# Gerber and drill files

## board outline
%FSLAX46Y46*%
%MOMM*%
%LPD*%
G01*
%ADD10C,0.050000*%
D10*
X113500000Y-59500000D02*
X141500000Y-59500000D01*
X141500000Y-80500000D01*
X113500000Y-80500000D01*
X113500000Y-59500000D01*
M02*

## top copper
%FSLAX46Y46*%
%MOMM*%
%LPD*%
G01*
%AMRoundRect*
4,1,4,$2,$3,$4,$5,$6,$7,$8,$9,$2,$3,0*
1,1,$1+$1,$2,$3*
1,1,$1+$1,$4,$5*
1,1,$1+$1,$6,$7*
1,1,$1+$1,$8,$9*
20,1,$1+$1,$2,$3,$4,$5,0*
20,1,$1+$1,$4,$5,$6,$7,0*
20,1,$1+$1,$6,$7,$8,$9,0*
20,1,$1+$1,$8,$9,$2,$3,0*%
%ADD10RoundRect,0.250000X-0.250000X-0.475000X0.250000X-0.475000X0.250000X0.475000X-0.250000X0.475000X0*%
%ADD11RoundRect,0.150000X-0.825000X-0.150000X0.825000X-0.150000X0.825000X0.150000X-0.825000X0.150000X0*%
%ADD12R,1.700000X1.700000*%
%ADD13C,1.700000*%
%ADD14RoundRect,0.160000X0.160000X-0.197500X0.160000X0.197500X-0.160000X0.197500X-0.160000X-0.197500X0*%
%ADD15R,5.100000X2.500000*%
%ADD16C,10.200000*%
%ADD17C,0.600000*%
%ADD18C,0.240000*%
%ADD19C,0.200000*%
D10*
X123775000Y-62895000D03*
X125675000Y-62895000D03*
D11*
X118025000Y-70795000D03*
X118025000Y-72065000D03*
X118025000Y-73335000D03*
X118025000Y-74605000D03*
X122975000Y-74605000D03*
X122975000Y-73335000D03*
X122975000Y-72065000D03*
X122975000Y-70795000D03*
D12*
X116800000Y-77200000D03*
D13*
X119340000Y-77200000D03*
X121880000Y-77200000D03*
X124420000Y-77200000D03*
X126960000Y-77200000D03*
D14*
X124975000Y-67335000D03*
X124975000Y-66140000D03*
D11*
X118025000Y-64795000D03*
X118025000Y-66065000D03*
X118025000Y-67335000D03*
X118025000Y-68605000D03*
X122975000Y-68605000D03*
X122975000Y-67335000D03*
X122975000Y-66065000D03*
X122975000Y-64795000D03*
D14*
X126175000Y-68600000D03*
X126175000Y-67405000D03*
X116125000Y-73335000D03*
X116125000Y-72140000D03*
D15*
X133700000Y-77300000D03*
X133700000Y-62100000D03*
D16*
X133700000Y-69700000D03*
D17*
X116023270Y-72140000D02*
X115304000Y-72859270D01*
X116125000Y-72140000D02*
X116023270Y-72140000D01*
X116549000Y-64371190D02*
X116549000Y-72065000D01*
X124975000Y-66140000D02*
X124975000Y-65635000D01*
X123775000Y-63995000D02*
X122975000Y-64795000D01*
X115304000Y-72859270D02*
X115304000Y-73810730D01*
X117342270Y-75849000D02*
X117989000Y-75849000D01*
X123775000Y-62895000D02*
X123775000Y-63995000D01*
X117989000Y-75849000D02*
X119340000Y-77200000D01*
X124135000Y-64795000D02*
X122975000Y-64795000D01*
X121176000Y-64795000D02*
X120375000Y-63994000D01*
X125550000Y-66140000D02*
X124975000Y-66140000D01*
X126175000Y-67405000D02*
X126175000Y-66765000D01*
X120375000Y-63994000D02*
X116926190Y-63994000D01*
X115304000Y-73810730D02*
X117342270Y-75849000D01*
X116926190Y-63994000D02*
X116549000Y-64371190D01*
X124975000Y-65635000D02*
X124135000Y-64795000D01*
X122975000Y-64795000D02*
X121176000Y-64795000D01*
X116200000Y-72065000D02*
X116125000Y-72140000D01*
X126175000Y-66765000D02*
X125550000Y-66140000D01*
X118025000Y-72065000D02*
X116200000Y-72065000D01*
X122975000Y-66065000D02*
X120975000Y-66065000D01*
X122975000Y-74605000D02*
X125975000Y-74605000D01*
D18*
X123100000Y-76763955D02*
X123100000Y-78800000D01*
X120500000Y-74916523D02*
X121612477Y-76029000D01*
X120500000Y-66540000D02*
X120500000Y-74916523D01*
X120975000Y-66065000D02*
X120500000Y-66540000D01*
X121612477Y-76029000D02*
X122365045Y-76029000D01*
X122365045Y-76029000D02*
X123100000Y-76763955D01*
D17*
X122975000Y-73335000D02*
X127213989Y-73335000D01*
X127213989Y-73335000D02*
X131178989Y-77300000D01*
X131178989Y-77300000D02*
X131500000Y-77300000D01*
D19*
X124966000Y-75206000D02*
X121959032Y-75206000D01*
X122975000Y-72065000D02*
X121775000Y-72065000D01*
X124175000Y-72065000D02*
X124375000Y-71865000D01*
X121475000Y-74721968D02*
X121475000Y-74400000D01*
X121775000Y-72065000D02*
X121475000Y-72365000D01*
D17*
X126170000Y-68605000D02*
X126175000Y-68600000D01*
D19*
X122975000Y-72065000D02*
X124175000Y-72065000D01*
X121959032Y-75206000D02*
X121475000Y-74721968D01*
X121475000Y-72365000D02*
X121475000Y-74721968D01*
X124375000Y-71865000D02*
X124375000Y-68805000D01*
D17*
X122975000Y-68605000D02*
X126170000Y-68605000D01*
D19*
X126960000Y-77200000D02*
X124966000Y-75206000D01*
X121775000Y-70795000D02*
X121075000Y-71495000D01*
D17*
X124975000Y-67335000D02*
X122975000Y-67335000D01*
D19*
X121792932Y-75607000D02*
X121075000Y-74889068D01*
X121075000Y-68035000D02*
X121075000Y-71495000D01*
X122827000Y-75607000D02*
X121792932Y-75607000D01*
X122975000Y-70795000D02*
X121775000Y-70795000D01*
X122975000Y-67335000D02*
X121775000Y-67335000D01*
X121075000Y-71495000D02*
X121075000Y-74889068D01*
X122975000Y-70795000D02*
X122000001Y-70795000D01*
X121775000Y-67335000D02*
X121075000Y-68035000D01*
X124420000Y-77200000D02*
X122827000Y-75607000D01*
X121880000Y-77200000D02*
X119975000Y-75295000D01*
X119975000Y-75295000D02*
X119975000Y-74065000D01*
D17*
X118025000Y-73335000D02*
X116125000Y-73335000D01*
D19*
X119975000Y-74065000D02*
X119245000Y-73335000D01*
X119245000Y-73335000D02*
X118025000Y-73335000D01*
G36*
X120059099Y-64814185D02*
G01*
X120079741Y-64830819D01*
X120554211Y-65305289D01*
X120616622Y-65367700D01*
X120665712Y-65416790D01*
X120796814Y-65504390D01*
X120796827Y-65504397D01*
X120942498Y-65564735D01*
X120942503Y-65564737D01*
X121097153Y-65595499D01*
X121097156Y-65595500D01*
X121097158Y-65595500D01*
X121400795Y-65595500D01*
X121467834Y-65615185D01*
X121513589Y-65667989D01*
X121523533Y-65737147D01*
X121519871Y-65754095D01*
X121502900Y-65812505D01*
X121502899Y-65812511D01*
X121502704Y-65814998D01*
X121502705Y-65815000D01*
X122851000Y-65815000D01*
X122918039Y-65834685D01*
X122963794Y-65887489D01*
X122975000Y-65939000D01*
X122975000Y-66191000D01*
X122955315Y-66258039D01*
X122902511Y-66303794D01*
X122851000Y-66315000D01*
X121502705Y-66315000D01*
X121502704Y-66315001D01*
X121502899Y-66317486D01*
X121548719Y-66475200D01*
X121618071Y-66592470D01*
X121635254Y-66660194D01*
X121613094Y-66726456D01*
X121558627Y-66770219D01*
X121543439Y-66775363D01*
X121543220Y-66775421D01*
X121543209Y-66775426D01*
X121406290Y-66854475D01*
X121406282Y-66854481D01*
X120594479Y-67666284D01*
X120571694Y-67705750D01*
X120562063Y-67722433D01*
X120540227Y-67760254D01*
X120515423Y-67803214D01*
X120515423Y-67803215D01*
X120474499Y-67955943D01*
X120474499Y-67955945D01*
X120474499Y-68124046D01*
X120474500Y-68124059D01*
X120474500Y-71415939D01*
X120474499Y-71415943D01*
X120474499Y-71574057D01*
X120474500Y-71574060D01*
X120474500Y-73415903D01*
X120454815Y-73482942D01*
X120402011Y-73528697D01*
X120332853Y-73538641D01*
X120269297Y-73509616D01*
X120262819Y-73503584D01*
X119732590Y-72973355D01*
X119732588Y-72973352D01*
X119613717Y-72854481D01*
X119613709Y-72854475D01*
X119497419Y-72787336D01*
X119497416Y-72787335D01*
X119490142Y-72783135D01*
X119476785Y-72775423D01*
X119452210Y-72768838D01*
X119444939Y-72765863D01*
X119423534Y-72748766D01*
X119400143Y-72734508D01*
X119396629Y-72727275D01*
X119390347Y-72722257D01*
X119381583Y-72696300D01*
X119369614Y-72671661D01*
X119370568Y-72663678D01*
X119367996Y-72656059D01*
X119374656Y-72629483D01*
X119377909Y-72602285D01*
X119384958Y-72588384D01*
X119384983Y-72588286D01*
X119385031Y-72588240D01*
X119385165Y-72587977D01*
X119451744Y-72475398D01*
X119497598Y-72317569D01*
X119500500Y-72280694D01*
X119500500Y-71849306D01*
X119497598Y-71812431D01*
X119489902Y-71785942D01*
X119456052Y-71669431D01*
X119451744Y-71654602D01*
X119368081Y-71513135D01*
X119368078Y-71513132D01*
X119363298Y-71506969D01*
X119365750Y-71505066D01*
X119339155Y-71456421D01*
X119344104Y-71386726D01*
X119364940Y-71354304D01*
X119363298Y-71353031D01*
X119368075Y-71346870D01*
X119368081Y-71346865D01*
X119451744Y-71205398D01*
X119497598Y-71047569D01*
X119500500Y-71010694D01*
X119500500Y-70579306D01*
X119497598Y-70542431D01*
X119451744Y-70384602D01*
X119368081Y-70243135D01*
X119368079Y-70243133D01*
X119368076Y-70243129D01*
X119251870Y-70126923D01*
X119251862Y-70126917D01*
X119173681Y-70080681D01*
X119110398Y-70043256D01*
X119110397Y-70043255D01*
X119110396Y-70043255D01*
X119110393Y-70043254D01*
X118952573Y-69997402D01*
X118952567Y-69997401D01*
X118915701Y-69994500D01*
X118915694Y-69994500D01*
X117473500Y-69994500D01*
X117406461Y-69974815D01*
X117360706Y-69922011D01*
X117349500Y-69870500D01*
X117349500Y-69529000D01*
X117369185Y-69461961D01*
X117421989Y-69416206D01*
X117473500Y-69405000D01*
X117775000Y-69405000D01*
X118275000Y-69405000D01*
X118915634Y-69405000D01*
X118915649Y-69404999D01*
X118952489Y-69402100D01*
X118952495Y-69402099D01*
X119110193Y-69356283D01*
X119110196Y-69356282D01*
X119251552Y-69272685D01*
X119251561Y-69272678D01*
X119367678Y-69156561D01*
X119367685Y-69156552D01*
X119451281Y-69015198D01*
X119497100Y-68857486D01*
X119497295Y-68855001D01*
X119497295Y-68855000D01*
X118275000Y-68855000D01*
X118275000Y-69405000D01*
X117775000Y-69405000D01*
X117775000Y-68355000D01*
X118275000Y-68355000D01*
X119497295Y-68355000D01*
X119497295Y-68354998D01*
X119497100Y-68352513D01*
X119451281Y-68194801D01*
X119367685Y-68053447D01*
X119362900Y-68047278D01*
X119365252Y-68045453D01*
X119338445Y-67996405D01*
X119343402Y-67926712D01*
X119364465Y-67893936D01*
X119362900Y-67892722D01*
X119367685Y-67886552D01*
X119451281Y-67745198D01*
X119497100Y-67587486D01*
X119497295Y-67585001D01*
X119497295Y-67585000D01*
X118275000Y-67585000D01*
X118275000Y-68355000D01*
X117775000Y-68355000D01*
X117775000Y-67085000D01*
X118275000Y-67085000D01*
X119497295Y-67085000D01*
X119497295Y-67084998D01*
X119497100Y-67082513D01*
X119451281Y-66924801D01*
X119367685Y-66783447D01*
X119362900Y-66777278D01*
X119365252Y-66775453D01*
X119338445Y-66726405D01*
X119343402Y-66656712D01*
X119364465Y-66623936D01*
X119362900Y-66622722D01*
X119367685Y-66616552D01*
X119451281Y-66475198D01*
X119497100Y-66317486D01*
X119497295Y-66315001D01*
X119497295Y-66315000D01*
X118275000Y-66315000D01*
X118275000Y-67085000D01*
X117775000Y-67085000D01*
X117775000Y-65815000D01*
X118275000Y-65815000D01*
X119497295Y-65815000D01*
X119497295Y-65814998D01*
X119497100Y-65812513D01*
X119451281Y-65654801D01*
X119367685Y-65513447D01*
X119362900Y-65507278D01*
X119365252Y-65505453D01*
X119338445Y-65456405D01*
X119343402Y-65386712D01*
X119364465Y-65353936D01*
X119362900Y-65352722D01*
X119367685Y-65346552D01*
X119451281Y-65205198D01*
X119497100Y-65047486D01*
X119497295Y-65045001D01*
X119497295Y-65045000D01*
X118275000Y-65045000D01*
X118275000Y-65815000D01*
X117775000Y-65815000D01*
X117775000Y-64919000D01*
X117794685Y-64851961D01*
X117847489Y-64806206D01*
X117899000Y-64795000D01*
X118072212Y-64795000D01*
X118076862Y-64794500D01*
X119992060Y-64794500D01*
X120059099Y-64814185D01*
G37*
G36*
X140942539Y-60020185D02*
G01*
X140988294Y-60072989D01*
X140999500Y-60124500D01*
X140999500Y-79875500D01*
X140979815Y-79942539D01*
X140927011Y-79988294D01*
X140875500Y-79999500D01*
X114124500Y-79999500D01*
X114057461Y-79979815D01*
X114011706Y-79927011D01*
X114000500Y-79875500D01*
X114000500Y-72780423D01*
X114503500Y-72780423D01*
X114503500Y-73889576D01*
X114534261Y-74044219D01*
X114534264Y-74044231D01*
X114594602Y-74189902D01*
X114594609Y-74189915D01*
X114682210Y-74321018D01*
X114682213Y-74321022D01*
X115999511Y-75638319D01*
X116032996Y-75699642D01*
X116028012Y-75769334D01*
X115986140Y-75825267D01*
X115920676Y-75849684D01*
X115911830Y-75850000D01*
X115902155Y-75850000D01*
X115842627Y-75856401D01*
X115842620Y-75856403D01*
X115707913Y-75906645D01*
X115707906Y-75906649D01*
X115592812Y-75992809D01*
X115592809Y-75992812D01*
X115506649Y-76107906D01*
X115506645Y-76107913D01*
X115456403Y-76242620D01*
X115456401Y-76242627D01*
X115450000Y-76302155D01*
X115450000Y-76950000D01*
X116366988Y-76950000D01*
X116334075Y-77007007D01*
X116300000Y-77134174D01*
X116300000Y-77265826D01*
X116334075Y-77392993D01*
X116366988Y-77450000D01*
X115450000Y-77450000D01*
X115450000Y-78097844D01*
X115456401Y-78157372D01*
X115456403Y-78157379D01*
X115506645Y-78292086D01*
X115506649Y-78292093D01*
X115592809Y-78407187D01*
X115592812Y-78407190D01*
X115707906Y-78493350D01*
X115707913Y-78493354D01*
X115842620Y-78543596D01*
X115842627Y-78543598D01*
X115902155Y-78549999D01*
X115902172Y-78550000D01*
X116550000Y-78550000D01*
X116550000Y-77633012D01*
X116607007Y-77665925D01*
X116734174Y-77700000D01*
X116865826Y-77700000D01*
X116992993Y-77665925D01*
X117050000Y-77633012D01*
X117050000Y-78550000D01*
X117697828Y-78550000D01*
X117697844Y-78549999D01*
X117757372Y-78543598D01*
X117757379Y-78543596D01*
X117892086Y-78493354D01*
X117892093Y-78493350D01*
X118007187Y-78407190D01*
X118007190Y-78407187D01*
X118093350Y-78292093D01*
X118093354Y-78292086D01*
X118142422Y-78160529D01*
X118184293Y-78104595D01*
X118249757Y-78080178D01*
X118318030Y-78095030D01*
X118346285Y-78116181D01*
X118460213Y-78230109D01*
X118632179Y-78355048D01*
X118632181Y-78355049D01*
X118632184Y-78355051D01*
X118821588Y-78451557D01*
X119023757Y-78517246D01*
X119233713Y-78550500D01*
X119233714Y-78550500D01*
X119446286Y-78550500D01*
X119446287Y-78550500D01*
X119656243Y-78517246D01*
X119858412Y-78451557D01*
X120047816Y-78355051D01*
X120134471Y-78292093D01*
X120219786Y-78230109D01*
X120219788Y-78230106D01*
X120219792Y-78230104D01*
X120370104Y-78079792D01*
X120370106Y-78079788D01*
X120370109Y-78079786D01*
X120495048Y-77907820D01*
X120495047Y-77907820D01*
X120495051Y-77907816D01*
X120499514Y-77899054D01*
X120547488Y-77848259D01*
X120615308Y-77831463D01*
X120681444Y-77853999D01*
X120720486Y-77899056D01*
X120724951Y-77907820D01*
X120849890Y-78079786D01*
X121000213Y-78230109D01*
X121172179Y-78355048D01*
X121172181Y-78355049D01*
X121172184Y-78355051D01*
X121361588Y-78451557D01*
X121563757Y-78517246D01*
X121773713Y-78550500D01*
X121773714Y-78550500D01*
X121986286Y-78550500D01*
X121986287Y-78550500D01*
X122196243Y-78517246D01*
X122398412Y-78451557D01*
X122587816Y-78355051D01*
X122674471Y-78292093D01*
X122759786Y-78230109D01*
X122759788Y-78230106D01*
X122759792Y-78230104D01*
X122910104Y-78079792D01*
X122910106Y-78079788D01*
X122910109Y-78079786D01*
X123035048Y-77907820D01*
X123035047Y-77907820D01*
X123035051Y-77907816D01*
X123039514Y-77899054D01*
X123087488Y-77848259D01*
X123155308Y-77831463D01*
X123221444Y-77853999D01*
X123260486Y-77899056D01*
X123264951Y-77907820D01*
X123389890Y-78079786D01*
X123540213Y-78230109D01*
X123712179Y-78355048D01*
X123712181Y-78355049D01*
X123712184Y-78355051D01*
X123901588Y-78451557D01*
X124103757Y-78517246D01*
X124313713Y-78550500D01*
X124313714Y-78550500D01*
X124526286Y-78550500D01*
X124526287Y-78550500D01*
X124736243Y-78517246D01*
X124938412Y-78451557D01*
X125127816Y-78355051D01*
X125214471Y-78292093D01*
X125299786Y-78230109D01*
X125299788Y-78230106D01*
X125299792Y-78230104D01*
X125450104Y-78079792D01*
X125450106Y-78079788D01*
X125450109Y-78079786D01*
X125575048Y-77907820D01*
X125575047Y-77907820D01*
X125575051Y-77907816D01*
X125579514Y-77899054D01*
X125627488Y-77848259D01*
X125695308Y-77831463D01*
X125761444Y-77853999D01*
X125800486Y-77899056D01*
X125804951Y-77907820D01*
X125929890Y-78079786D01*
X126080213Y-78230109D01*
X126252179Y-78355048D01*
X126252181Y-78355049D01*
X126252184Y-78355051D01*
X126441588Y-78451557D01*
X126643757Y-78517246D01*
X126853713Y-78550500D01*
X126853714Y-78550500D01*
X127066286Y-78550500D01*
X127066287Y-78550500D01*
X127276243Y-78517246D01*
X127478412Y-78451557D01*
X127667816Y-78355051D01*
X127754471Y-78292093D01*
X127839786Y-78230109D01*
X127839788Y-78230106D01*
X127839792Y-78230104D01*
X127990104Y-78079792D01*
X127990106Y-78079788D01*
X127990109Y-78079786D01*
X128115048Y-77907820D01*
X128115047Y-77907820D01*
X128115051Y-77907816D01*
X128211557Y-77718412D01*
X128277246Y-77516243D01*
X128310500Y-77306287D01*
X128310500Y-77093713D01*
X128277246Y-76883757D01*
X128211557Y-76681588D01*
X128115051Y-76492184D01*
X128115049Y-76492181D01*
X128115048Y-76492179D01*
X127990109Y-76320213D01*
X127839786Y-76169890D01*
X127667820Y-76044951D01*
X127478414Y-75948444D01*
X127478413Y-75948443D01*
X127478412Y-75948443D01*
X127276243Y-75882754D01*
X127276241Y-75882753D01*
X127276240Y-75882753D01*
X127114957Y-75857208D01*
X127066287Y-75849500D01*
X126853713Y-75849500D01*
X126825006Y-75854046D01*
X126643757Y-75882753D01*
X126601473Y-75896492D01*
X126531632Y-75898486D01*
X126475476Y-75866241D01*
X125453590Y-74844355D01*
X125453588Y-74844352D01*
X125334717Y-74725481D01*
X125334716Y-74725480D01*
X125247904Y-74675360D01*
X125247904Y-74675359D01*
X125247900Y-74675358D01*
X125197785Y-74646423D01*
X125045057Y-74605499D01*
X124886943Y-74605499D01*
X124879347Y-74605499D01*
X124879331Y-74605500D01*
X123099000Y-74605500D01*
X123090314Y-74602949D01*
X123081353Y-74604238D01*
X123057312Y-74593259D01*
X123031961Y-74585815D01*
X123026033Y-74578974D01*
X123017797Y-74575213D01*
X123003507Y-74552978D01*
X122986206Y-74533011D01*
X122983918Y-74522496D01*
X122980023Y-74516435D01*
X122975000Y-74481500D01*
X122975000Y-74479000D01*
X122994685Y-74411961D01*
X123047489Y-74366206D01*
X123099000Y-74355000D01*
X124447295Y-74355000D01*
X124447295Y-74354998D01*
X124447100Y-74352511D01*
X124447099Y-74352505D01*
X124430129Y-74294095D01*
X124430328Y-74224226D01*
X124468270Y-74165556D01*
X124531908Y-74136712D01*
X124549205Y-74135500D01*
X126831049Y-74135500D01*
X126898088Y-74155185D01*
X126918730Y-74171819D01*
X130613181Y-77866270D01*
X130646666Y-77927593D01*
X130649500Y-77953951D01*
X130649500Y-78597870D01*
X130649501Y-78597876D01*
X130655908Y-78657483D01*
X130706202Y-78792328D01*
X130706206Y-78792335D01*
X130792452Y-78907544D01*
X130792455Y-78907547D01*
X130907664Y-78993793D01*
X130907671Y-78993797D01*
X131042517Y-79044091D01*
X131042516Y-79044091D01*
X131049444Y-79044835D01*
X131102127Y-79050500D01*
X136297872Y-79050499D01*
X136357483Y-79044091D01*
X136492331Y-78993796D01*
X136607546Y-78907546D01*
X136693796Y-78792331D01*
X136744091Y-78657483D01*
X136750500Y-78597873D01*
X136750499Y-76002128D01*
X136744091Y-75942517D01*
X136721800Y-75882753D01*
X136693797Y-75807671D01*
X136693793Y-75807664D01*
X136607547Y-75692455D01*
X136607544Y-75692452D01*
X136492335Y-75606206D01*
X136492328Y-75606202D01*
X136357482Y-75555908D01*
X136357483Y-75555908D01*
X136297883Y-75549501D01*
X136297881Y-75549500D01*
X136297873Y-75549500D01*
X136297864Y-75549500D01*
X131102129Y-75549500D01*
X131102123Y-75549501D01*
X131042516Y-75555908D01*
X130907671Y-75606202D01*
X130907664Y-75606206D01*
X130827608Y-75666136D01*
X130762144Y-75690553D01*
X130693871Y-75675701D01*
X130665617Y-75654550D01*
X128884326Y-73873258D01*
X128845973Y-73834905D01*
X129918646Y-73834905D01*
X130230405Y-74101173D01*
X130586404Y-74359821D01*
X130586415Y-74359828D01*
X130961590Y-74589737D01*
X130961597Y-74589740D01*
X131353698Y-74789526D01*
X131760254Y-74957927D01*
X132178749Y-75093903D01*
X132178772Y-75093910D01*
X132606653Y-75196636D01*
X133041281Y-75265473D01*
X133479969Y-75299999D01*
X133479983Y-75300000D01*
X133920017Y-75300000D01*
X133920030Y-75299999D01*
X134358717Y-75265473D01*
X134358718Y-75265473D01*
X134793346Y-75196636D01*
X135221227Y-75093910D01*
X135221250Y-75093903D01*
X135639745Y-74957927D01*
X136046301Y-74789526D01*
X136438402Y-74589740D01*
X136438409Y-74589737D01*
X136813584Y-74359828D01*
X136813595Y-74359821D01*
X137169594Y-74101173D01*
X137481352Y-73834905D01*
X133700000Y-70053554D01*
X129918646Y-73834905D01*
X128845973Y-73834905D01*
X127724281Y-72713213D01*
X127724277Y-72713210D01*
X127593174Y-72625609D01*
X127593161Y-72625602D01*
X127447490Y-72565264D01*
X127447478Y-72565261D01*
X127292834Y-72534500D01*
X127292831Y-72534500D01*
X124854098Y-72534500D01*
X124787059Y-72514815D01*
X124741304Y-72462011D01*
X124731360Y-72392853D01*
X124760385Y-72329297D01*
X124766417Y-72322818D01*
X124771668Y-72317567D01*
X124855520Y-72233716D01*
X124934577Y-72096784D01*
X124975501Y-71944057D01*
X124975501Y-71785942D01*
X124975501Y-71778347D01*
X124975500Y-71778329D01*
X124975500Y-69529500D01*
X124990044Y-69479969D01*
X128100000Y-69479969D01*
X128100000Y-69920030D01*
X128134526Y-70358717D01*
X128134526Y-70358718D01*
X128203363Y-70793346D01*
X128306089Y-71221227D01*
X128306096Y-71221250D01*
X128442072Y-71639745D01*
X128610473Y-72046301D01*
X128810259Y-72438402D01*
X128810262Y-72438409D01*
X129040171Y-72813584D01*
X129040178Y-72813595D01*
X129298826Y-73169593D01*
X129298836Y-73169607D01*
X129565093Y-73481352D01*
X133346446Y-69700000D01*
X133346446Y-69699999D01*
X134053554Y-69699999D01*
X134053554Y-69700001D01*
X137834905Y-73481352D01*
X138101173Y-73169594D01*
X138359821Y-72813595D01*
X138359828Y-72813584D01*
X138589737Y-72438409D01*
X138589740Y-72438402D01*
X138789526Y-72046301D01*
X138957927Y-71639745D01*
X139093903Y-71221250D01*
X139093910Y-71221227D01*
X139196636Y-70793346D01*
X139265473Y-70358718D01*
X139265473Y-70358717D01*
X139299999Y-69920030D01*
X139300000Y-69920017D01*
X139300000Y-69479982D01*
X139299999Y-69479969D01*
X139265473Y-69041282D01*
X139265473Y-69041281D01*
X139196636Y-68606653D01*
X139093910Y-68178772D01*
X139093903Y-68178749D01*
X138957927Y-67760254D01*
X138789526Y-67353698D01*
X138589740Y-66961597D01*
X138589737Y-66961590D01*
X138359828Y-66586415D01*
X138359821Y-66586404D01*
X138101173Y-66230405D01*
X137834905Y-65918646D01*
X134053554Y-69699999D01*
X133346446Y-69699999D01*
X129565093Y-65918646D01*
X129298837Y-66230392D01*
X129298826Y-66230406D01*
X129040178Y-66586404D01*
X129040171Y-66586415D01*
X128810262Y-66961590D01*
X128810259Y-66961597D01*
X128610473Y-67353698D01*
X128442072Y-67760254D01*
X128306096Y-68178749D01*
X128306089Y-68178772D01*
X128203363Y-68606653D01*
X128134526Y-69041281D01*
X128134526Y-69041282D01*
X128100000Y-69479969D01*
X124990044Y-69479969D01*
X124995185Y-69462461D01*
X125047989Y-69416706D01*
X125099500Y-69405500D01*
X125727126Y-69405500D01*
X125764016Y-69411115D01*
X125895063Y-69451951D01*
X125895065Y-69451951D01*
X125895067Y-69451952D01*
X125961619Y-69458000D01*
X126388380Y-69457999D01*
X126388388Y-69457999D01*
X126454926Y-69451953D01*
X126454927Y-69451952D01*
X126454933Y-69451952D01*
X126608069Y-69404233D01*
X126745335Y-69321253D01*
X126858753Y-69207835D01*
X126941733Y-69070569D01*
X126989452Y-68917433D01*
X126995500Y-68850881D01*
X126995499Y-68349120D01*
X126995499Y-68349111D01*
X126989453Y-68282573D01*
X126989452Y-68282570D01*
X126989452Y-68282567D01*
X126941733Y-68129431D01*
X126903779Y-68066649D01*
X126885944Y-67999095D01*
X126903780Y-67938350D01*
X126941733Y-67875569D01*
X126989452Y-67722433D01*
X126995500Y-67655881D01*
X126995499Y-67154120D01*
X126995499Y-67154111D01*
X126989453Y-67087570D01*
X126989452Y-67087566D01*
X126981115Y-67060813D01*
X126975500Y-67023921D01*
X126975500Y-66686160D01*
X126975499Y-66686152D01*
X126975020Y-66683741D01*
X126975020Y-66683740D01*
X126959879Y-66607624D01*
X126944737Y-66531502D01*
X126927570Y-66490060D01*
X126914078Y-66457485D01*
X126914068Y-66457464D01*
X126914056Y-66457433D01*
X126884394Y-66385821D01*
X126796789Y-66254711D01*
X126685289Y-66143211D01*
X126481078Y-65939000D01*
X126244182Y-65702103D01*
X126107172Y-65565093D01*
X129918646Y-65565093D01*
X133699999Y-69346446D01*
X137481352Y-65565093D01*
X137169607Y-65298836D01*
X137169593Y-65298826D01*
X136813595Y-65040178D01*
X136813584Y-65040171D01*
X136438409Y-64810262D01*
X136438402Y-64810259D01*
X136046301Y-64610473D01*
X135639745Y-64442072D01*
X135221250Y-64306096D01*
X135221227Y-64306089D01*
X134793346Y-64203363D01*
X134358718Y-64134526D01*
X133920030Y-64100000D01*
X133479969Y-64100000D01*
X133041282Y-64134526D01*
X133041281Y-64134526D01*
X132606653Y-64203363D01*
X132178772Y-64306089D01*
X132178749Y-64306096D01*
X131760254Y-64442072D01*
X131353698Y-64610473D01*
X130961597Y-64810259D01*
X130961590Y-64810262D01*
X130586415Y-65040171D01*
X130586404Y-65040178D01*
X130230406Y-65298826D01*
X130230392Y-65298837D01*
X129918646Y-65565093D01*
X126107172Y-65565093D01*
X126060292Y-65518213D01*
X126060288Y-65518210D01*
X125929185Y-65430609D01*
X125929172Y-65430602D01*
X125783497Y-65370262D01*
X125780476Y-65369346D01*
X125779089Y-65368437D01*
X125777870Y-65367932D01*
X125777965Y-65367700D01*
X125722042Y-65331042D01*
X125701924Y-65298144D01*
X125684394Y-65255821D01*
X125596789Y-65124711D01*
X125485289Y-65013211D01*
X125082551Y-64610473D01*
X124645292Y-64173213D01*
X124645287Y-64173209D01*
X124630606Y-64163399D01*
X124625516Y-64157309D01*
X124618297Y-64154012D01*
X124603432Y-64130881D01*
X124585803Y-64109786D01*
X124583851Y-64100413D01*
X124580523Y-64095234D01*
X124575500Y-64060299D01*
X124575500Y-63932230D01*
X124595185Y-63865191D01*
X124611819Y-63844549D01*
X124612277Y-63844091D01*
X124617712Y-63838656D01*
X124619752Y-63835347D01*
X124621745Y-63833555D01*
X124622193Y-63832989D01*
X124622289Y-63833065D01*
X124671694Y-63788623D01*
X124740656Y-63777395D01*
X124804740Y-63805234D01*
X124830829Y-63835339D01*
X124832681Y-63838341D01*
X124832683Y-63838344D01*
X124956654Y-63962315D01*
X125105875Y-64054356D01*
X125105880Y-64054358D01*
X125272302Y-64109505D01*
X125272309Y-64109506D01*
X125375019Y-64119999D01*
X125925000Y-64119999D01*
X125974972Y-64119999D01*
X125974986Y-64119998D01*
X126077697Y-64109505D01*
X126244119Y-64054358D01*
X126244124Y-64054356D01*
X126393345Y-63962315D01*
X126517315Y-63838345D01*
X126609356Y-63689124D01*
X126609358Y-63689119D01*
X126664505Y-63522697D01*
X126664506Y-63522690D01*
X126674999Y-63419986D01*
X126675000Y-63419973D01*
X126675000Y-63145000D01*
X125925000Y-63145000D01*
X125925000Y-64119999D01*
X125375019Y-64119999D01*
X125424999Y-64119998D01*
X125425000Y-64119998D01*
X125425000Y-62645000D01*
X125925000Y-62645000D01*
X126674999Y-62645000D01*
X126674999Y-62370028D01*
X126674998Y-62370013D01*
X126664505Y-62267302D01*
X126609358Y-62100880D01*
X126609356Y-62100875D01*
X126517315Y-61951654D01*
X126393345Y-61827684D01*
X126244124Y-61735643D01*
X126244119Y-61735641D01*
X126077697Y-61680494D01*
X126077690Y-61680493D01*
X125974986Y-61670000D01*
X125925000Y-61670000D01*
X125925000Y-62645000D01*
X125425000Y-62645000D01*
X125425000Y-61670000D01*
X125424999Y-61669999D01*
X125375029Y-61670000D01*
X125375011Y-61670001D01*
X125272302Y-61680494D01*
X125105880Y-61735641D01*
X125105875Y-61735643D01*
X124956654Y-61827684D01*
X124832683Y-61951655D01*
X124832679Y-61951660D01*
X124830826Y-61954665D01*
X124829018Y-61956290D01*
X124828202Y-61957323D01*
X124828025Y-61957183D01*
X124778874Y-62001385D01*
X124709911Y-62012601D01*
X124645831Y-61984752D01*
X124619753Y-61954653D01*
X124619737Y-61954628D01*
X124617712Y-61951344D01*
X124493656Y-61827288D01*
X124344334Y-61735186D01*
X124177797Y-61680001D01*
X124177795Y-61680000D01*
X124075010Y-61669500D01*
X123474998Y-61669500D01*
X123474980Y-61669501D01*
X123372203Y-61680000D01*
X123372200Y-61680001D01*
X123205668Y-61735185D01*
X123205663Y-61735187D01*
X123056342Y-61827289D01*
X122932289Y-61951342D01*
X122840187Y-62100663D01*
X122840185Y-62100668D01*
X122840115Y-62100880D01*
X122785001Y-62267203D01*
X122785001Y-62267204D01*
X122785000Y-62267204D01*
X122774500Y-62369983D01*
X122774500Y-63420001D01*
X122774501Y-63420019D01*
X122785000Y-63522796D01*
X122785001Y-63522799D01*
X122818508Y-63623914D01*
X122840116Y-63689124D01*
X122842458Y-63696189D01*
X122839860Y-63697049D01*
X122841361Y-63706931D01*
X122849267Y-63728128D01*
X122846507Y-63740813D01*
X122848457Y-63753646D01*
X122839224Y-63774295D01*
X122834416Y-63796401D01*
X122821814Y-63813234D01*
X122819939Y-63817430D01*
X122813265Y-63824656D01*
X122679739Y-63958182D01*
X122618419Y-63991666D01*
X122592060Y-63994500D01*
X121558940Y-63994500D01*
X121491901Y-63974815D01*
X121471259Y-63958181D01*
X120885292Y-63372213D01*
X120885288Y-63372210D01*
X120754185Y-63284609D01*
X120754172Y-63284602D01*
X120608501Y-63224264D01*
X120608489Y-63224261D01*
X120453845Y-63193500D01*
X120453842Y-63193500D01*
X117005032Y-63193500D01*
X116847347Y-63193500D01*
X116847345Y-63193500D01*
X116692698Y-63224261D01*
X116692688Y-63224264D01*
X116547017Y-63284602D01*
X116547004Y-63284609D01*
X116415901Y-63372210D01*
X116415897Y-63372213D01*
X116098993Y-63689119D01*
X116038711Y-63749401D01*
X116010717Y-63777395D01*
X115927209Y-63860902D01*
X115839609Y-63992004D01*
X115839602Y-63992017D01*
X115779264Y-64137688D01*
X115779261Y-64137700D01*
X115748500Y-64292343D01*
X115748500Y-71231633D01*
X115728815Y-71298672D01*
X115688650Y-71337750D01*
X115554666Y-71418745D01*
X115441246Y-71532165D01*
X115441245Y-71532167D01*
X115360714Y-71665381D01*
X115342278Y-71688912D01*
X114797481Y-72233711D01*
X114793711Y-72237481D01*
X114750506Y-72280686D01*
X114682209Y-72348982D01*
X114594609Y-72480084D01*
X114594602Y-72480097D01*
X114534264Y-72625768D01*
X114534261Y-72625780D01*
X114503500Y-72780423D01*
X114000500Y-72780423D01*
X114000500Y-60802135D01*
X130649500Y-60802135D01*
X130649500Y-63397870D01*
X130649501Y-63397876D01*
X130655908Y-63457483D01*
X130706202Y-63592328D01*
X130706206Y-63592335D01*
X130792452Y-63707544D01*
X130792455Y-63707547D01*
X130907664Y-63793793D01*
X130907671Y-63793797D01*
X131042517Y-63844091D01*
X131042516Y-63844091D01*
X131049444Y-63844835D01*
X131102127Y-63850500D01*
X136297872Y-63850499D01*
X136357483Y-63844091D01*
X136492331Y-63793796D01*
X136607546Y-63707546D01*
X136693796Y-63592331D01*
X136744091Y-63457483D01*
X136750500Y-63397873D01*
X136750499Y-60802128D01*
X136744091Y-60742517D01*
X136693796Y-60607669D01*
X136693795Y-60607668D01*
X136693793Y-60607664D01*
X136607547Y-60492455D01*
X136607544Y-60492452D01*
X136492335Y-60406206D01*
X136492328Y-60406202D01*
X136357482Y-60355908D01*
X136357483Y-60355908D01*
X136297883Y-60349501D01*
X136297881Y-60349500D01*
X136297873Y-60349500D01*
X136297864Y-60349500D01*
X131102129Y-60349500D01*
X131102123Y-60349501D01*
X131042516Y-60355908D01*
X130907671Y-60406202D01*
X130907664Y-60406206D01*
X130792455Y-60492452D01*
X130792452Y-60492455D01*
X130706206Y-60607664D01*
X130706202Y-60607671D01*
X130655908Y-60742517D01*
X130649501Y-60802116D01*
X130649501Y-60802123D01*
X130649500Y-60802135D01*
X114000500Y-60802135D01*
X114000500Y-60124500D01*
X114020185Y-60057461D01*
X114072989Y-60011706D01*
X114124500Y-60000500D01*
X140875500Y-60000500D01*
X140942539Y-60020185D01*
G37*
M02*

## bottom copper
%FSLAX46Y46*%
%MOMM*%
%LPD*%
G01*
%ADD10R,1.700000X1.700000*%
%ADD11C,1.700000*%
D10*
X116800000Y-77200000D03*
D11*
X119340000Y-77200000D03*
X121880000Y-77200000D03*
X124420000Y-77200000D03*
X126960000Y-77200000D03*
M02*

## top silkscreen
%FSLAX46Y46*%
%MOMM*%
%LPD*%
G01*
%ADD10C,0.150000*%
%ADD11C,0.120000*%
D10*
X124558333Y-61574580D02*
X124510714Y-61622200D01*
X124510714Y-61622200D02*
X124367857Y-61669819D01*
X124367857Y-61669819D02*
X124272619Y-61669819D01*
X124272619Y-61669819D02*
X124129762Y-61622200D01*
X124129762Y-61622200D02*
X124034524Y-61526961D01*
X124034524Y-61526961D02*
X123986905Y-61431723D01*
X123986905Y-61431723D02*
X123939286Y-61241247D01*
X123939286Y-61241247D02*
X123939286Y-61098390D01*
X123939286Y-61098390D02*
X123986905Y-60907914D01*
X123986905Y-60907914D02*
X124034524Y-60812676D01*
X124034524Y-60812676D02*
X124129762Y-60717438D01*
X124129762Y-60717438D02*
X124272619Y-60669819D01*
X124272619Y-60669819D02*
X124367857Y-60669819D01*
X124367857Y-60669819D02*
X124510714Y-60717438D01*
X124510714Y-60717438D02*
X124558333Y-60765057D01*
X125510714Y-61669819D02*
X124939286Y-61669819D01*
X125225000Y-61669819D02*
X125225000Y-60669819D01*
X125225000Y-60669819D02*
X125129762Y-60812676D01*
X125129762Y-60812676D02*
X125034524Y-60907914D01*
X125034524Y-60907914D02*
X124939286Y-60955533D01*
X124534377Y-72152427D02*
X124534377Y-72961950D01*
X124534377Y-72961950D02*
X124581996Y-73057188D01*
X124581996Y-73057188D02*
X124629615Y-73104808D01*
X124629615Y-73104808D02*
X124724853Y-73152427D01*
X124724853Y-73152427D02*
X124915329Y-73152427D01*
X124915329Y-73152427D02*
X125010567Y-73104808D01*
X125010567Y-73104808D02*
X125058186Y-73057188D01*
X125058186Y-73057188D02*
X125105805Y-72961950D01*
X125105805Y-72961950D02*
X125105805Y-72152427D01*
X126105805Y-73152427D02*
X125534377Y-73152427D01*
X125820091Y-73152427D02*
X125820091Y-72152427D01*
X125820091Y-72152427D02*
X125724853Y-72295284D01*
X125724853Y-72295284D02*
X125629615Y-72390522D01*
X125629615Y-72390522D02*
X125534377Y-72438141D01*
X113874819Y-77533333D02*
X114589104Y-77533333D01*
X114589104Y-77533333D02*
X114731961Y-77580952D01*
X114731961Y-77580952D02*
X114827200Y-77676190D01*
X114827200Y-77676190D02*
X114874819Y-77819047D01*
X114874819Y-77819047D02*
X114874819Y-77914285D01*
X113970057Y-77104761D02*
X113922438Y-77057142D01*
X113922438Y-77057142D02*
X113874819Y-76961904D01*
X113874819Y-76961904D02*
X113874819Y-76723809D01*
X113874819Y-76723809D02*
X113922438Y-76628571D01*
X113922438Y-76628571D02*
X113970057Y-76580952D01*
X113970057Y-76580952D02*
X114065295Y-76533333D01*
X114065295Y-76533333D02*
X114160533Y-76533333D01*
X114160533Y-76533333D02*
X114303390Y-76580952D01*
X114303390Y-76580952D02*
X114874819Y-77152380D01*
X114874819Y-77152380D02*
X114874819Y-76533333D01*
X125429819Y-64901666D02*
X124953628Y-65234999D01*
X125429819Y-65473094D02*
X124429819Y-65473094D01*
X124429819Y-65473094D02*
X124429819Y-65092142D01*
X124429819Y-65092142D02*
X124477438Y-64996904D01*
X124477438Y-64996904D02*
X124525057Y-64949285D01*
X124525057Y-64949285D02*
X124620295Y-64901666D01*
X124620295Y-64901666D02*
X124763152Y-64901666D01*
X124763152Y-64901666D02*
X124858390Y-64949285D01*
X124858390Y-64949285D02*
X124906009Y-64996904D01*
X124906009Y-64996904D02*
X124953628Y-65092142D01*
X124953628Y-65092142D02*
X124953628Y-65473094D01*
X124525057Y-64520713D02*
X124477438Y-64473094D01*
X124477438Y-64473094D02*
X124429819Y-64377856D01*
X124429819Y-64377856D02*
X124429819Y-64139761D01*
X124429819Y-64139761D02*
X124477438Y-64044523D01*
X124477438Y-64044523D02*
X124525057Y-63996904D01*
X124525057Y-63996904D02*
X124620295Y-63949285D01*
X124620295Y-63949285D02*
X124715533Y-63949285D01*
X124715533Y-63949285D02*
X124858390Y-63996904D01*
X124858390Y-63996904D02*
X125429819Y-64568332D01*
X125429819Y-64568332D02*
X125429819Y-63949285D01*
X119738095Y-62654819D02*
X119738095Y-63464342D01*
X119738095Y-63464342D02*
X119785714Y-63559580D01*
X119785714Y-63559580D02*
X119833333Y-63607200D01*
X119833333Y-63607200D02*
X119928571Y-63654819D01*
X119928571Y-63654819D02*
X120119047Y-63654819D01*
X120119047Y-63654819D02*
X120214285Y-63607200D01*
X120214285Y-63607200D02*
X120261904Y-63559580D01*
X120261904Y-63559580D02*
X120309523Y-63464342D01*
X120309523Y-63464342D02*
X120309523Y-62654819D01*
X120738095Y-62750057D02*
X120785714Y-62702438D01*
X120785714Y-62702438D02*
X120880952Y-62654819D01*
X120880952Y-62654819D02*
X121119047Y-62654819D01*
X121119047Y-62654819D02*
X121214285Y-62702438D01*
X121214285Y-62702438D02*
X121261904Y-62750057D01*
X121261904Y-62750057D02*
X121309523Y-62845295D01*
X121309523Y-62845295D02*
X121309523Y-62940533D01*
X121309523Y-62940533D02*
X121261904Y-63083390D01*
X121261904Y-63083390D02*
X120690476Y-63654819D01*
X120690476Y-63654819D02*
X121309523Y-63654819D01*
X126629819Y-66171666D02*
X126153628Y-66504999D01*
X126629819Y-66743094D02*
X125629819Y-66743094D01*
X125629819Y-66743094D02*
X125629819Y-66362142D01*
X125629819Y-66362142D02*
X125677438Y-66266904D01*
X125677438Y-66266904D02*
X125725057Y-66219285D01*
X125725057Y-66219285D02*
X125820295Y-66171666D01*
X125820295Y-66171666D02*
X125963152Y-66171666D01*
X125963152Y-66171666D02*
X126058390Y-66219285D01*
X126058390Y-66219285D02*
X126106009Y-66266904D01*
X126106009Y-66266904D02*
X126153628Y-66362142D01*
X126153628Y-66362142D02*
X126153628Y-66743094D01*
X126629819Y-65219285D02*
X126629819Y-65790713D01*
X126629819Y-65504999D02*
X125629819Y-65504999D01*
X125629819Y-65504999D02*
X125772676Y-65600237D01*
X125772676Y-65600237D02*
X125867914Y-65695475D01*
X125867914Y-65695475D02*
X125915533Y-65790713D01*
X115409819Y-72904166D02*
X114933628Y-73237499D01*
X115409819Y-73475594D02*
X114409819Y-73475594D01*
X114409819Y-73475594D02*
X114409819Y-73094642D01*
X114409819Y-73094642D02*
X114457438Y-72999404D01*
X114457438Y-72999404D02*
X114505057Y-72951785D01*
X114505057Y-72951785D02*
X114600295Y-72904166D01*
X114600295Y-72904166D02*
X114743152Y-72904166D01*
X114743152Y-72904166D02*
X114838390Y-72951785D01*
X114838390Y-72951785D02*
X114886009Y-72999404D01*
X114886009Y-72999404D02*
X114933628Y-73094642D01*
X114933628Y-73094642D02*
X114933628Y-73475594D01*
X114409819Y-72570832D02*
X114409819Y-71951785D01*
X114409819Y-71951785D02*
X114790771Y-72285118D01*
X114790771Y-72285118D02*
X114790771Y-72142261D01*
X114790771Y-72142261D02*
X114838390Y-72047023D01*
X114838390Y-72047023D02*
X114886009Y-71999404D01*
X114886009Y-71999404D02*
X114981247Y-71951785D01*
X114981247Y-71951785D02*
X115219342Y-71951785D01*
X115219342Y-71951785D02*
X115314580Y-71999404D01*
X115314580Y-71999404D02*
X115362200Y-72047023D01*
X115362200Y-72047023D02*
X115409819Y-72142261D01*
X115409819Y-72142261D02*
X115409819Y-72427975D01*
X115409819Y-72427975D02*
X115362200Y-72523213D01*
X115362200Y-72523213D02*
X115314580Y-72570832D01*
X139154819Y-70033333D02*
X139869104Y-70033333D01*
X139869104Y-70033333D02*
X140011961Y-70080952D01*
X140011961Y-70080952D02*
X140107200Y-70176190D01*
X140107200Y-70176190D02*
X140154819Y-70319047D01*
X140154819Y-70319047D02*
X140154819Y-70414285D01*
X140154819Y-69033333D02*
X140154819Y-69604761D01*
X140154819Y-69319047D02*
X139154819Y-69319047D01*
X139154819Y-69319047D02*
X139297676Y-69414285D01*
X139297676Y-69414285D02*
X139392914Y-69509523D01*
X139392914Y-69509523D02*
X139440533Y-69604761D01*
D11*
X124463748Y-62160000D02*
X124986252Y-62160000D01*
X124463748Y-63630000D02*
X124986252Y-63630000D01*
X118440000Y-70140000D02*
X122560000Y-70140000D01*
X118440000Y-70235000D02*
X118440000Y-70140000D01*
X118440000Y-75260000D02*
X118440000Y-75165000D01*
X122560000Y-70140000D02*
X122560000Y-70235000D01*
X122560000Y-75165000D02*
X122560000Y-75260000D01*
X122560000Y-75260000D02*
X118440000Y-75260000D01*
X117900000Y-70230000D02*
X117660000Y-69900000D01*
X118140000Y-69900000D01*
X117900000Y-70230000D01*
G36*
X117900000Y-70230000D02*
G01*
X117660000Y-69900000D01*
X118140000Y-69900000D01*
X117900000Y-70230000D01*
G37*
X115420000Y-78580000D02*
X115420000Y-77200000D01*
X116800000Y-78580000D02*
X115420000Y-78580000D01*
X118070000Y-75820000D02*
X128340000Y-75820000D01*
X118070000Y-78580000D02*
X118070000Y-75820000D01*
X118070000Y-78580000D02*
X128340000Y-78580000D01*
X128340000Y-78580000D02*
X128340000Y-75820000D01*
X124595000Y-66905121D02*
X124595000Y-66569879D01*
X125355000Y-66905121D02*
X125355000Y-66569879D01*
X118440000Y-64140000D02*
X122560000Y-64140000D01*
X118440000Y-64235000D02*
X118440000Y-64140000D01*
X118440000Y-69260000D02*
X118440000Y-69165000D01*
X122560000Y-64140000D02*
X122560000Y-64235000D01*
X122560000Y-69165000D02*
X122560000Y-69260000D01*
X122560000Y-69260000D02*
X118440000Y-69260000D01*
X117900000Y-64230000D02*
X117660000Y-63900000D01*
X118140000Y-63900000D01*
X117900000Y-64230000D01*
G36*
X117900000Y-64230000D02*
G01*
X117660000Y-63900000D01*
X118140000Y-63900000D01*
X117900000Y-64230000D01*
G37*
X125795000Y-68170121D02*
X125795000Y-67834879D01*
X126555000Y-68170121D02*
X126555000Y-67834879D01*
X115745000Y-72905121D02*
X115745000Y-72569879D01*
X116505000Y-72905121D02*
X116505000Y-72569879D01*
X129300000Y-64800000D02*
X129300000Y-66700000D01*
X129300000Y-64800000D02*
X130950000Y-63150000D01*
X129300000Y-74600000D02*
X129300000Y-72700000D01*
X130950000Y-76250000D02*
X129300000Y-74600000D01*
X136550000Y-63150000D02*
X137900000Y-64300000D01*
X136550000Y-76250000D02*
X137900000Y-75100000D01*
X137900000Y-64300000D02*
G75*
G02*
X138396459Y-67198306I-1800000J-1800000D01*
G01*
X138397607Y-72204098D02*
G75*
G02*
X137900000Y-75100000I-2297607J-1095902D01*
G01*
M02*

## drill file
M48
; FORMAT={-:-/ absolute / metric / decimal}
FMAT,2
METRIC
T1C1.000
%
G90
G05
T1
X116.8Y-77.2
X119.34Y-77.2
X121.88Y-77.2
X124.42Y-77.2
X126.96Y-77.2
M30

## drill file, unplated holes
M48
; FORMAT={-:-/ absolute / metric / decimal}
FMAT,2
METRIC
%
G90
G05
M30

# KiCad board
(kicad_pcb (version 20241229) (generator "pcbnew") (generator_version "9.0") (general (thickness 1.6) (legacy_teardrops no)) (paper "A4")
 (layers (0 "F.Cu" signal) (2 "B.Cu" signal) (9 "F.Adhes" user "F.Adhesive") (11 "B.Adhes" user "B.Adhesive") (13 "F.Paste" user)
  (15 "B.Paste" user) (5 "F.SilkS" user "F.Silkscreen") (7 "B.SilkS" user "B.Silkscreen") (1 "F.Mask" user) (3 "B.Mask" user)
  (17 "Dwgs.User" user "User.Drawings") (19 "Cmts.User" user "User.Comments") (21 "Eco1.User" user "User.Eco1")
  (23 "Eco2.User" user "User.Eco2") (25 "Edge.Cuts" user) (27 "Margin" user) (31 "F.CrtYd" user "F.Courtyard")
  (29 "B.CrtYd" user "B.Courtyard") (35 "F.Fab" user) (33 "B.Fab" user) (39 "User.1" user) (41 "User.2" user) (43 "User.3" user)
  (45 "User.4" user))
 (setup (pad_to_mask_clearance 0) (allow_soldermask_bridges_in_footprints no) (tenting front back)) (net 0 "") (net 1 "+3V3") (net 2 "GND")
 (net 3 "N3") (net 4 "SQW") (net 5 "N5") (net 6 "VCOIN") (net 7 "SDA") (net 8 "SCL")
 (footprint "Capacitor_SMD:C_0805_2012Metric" (layer "F.Cu") (at 124.725 62.895)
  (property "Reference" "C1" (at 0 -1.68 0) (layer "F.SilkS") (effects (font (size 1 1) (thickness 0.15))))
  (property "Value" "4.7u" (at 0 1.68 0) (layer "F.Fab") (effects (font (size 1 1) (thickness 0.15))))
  (fp_line (start -0.261252 -0.735) (end 0.261252 -0.735) (stroke (width 0.12) (type solid)) (layer "F.SilkS"))
  (fp_line (start -0.261252 0.735) (end 0.261252 0.735) (stroke (width 0.12) (type solid)) (layer "F.SilkS"))
  (pad "1" smd roundrect (at -0.95 0) (size 1 1.45) (layers "F.Cu" "F.Mask" "F.Paste") (roundrect_rratio 0.25) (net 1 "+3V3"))
  (pad "2" smd roundrect (at 0.95 0) (size 1 1.45) (layers "F.Cu" "F.Mask" "F.Paste") (roundrect_rratio 0.25) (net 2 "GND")))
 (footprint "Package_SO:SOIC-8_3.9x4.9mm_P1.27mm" (layer "F.Cu") (at 120.5 72.7)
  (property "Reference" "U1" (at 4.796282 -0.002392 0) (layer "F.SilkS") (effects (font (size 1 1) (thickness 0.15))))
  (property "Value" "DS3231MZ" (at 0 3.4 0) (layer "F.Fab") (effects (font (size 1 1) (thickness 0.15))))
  (fp_line (start -2.06 -2.56) (end 2.06 -2.56) (stroke (width 0.12) (type solid)) (layer "F.SilkS"))
  (fp_line (start -2.06 -2.465) (end -2.06 -2.56) (stroke (width 0.12) (type solid)) (layer "F.SilkS"))
  (fp_line (start -2.06 2.56) (end -2.06 2.465) (stroke (width 0.12) (type solid)) (layer "F.SilkS"))
  (fp_line (start 2.06 -2.56) (end 2.06 -2.465) (stroke (width 0.12) (type solid)) (layer "F.SilkS"))
  (fp_line (start 2.06 2.465) (end 2.06 2.56) (stroke (width 0.12) (type solid)) (layer "F.SilkS"))
  (fp_line (start 2.06 2.56) (end -2.06 2.56) (stroke (width 0.12) (type solid)) (layer "F.SilkS"))
  (fp_poly (pts (xy -2.6 -2.47) (xy -2.84 -2.8) (xy -2.36 -2.8)) (stroke (width 0.12) (type solid)) (fill yes) (layer "F.SilkS"))
  (pad "1" smd roundrect (at -2.475 -1.905) (size 1.95 0.6) (layers "F.Cu" "F.Mask" "F.Paste") (roundrect_rratio 0.25) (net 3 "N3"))
  (pad "2" smd roundrect (at -2.475 -0.635) (size 1.95 0.6) (layers "F.Cu" "F.Mask" "F.Paste") (roundrect_rratio 0.25) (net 1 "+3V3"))
  (pad "3" smd roundrect (at -2.475 0.635) (size 1.95 0.6) (layers "F.Cu" "F.Mask" "F.Paste") (roundrect_rratio 0.25) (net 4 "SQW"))
  (pad "4" smd roundrect (at -2.475 1.905) (size 1.95 0.6) (layers "F.Cu" "F.Mask" "F.Paste") (roundrect_rratio 0.25) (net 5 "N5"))
  (pad "5" smd roundrect (at 2.475 1.905) (size 1.95 0.6) (layers "F.Cu" "F.Mask" "F.Paste") (roundrect_rratio 0.25) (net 2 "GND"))
  (pad "6" smd roundrect (at 2.475 0.635) (size 1.95 0.6) (layers "F.Cu" "F.Mask" "F.Paste") (roundrect_rratio 0.25) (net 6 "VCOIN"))
  (pad "7" smd roundrect (at 2.475 -0.635) (size 1.95 0.6) (layers "F.Cu" "F.Mask" "F.Paste") (roundrect_rratio 0.25) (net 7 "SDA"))
  (pad "8" smd roundrect (at 2.475 -1.905) (size 1.95 0.6) (layers "F.Cu" "F.Mask" "F.Paste") (roundrect_rratio 0.25) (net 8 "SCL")))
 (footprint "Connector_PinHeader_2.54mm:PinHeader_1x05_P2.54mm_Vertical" (layer "F.Cu") (at 116.8 77.2 90)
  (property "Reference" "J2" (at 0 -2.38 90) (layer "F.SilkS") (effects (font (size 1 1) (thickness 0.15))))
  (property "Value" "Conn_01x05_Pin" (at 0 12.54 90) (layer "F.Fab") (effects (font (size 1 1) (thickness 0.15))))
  (fp_line (start -1.38 -1.38) (end 0 -1.38) (stroke (width 0.12) (type solid)) (layer "F.SilkS"))
  (fp_line (start -1.38 0) (end -1.38 -1.38) (stroke (width 0.12) (type solid)) (layer "F.SilkS"))
  (fp_line (start 1.38 1.27) (end 1.38 11.54) (stroke (width 0.12) (type solid)) (layer "F.SilkS"))
  (fp_line (start -1.38 1.27) (end 1.38 1.27) (stroke (width 0.12) (type solid)) (layer "F.SilkS"))
  (fp_line (start -1.38 1.27) (end -1.38 11.54) (stroke (width 0.12) (type solid)) (layer "F.SilkS"))
  (fp_line (start -1.38 11.54) (end 1.38 11.54) (stroke (width 0.12) (type solid)) (layer "F.SilkS"))
  (pad "1" thru_hole rect (at 0 0 90) (size 1.7 1.7) (drill 1) (layers "*.Cu" "*.Mask") (remove_unused_layers no) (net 2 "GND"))
  (pad "2" thru_hole circle (at 0 2.54 90) (size 1.7 1.7) (drill 1) (layers "*.Cu" "*.Mask") (remove_unused_layers no) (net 1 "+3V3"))
  (pad "3" thru_hole circle (at 0 5.08 90) (size 1.7 1.7) (drill 1) (layers "*.Cu" "*.Mask") (remove_unused_layers no) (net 4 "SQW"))
  (pad "4" thru_hole circle (at 0 7.62 90) (size 1.7 1.7) (drill 1) (layers "*.Cu" "*.Mask") (remove_unused_layers no) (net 8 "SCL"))
  (pad "5" thru_hole circle (at 0 10.16 90) (size 1.7 1.7) (drill 1) (layers "*.Cu" "*.Mask") (remove_unused_layers no) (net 7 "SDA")))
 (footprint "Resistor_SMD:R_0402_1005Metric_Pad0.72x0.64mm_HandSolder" (layer "F.Cu") (at 124.975 66.7375 90)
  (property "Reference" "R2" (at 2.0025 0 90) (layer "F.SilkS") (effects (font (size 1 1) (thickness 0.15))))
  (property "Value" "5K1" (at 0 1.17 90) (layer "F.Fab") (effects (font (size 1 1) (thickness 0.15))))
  (fp_line (start -0.167621 -0.38) (end 0.167621 -0.38) (stroke (width 0.12) (type solid)) (layer "F.SilkS"))
  (fp_line (start -0.167621 0.38) (end 0.167621 0.38) (stroke (width 0.12) (type solid)) (layer "F.SilkS"))
  (pad "1" smd roundrect (at -0.5975 0 90) (size 0.715 0.64) (layers "F.Cu" "F.Mask" "F.Paste") (roundrect_rratio 0.25) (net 8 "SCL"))
  (pad "2" smd roundrect (at 0.5975 0 90) (size 0.715 0.64) (layers "F.Cu" "F.Mask" "F.Paste") (roundrect_rratio 0.25) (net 1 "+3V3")))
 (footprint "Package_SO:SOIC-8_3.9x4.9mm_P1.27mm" (layer "F.Cu") (at 120.5 66.7)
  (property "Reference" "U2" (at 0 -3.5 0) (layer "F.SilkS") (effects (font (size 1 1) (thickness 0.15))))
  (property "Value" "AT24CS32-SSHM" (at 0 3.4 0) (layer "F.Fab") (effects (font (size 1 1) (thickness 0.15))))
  (fp_line (start -2.06 -2.56) (end 2.06 -2.56) (stroke (width 0.12) (type solid)) (layer "F.SilkS"))
  (fp_line (start -2.06 -2.465) (end -2.06 -2.56) (stroke (width 0.12) (type solid)) (layer "F.SilkS"))
  (fp_line (start -2.06 2.56) (end -2.06 2.465) (stroke (width 0.12) (type solid)) (layer "F.SilkS"))
  (fp_line (start 2.06 -2.56) (end 2.06 -2.465) (stroke (width 0.12) (type solid)) (layer "F.SilkS"))
  (fp_line (start 2.06 2.465) (end 2.06 2.56) (stroke (width 0.12) (type solid)) (layer "F.SilkS"))
  (fp_line (start 2.06 2.56) (end -2.06 2.56) (stroke (width 0.12) (type solid)) (layer "F.SilkS"))
  (fp_poly (pts (xy -2.6 -2.47) (xy -2.84 -2.8) (xy -2.36 -2.8)) (stroke (width 0.12) (type solid)) (fill yes) (layer "F.SilkS"))
  (pad "1" smd roundrect (at -2.475 -1.905) (size 1.95 0.6) (layers "F.Cu" "F.Mask" "F.Paste") (roundrect_rratio 0.25) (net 2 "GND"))
  (pad "2" smd roundrect (at -2.475 -0.635) (size 1.95 0.6) (layers "F.Cu" "F.Mask" "F.Paste") (roundrect_rratio 0.25) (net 2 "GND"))
  (pad "3" smd roundrect (at -2.475 0.635) (size 1.95 0.6) (layers "F.Cu" "F.Mask" "F.Paste") (roundrect_rratio 0.25) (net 2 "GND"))
  (pad "4" smd roundrect (at -2.475 1.905) (size 1.95 0.6) (layers "F.Cu" "F.Mask" "F.Paste") (roundrect_rratio 0.25) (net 2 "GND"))
  (pad "5" smd roundrect (at 2.475 1.905) (size 1.95 0.6) (layers "F.Cu" "F.Mask" "F.Paste") (roundrect_rratio 0.25) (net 7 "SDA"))
  (pad "6" smd roundrect (at 2.475 0.635) (size 1.95 0.6) (layers "F.Cu" "F.Mask" "F.Paste") (roundrect_rratio 0.25) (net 8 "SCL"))
  (pad "7" smd roundrect (at 2.475 -0.635) (size 1.95 0.6) (layers "F.Cu" "F.Mask" "F.Paste") (roundrect_rratio 0.25) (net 2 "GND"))
  (pad "8" smd roundrect (at 2.475 -1.905) (size 1.95 0.6) (layers "F.Cu" "F.Mask" "F.Paste") (roundrect_rratio 0.25) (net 1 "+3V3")))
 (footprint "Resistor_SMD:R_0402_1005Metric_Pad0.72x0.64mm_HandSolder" (layer "F.Cu") (at 126.175 68.0025 90)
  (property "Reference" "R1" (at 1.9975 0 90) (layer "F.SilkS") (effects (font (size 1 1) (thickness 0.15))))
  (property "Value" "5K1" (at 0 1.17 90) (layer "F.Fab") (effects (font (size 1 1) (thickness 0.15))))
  (fp_line (start -0.167621 -0.38) (end 0.167621 -0.38) (stroke (width 0.12) (type solid)) (layer "F.SilkS"))
  (fp_line (start -0.167621 0.38) (end 0.167621 0.38) (stroke (width 0.12) (type solid)) (layer "F.SilkS"))
  (pad "1" smd roundrect (at -0.5975 0 90) (size 0.715 0.64) (layers "F.Cu" "F.Mask" "F.Paste") (roundrect_rratio 0.25) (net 7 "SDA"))
  (pad "2" smd roundrect (at 0.5975 0 90) (size 0.715 0.64) (layers "F.Cu" "F.Mask" "F.Paste") (roundrect_rratio 0.25) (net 1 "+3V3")))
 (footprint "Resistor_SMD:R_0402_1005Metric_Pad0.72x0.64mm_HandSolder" (layer "F.Cu") (at 116.125 72.7375 90)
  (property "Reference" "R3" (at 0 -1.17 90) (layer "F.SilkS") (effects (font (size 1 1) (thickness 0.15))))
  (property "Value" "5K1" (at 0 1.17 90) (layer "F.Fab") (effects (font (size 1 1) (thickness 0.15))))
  (fp_line (start -0.167621 -0.38) (end 0.167621 -0.38) (stroke (width 0.12) (type solid)) (layer "F.SilkS"))
  (fp_line (start -0.167621 0.38) (end 0.167621 0.38) (stroke (width 0.12) (type solid)) (layer "F.SilkS"))
  (pad "1" smd roundrect (at -0.5975 0 90) (size 0.715 0.64) (layers "F.Cu" "F.Mask" "F.Paste") (roundrect_rratio 0.25) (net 4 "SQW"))
  (pad "2" smd roundrect (at 0.5975 0 90) (size 0.715 0.64) (layers "F.Cu" "F.Mask" "F.Paste") (roundrect_rratio 0.25) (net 1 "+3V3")))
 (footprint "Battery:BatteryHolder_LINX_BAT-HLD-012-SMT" (layer "F.Cu") (at 133.7 69.7 90)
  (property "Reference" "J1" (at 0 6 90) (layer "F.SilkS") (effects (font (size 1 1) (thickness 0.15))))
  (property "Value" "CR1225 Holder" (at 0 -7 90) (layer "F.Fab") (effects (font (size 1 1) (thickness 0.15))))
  (fp_line (start 4.9 -4.4) (end 3 -4.4) (stroke (width 0.12) (type solid)) (layer "F.SilkS"))
  (fp_line (start 4.9 -4.4) (end 6.55 -2.75) (stroke (width 0.12) (type solid)) (layer "F.SilkS"))
  (fp_line (start -4.9 -4.4) (end -3 -4.4) (stroke (width 0.12) (type solid)) (layer "F.SilkS"))
  (fp_line (start -6.55 -2.75) (end -4.9 -4.4) (stroke (width 0.12) (type solid)) (layer "F.SilkS"))
  (fp_line (start 6.55 2.85) (end 5.4 4.2) (stroke (width 0.12) (type solid)) (layer "F.SilkS"))
  (fp_line (start -6.55 2.85) (end -5.4 4.2) (stroke (width 0.12) (type solid)) (layer "F.SilkS"))
  (fp_arc (start 5.4 4.2) (mid 4.029781 4.909041) (end 2.501694 4.696459) (stroke (width 0.12) (type solid)) (layer "F.SilkS"))
  (fp_arc (start -2.504098 4.697607) (mid -4.031094 4.908816) (end -5.4 4.2) (stroke (width 0.12) (type solid)) (layer "F.SilkS"))
  (pad "1" smd rect (at -7.6 0 90) (size 2.5 5.1) (layers "F.Cu" "F.Mask" "F.Paste") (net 6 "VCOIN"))
  (pad "1" smd rect (at 7.6 0 90) (size 2.5 5.1) (layers "F.Cu" "F.Mask" "F.Paste") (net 6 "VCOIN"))
  (pad "2" smd circle (at 0 0 90) (size 10.2 10.2) (layers "F.Cu" "F.Mask") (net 2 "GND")))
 (gr_rect (start 113.5 59.5) (end 141.5 80.5) (stroke (width 0.05) (type default)) (fill no) (layer "Edge.Cuts"))
 (segment (start 116.02327 72.14) (end 115.304 72.85927) (width 0.6) (layer "F.Cu") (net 1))
 (segment (start 116.125 72.14) (end 116.02327 72.14) (width 0.6) (layer "F.Cu") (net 1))
 (segment (start 116.549 64.37119) (end 116.549 72.065) (width 0.6) (layer "F.Cu") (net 1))
 (segment (start 124.975 66.14) (end 124.975 65.635) (width 0.6) (layer "F.Cu") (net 1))
 (segment (start 123.775 63.995) (end 122.975 64.795) (width 0.6) (layer "F.Cu") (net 1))
 (segment (start 115.304 72.85927) (end 115.304 73.81073) (width 0.6) (layer "F.Cu") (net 1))
 (segment (start 117.34227 75.849) (end 117.989 75.849) (width 0.6) (layer "F.Cu") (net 1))
 (segment (start 123.775 62.895) (end 123.775 63.995) (width 0.6) (layer "F.Cu") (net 1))
 (segment (start 117.989 75.849) (end 119.34 77.2) (width 0.6) (layer "F.Cu") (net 1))
 (segment (start 124.135 64.795) (end 122.975 64.795) (width 0.6) (layer "F.Cu") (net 1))
 (segment (start 121.176 64.795) (end 120.375 63.994) (width 0.6) (layer "F.Cu") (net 1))
 (segment (start 125.55 66.14) (end 124.975 66.14) (width 0.6) (layer "F.Cu") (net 1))
 (segment (start 126.175 67.405) (end 126.175 66.765) (width 0.6) (layer "F.Cu") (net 1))
 (segment (start 120.375 63.994) (end 116.92619 63.994) (width 0.6) (layer "F.Cu") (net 1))
 (segment (start 115.304 73.81073) (end 117.34227 75.849) (width 0.6) (layer "F.Cu") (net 1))
 (segment (start 116.92619 63.994) (end 116.549 64.37119) (width 0.6) (layer "F.Cu") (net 1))
 (segment (start 124.975 65.635) (end 124.135 64.795) (width 0.6) (layer "F.Cu") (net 1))
 (segment (start 122.975 64.795) (end 121.176 64.795) (width 0.6) (layer "F.Cu") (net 1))
 (segment (start 116.2 72.065) (end 116.125 72.14) (width 0.6) (layer "F.Cu") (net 1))
 (segment (start 126.175 66.765) (end 125.55 66.14) (width 0.6) (layer "F.Cu") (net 1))
 (segment (start 118.025 72.065) (end 116.2 72.065) (width 0.6) (layer "F.Cu") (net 1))
 (segment (start 122.975 66.065) (end 120.975 66.065) (width 0.6) (layer "F.Cu") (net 2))
 (segment (start 122.975 74.605) (end 125.975 74.605) (width 0.6) (layer "F.Cu") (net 2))
 (segment (start 123.1 76.763955) (end 123.1 78.8) (width 0.24) (layer "F.Cu") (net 2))
 (segment (start 120.5 74.916523) (end 121.612477 76.029) (width 0.24) (layer "F.Cu") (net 2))
 (segment (start 120.5 66.54) (end 120.5 74.916523) (width 0.24) (layer "F.Cu") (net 2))
 (segment (start 120.975 66.065) (end 120.5 66.54) (width 0.24) (layer "F.Cu") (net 2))
 (segment (start 121.612477 76.029) (end 122.365045 76.029) (width 0.24) (layer "F.Cu") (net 2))
 (segment (start 122.365045 76.029) (end 123.1 76.763955) (width 0.24) (layer "F.Cu") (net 2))
 (segment (start 122.975 73.335) (end 127.213989 73.335) (width 0.6) (layer "F.Cu") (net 6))
 (segment (start 127.213989 73.335) (end 131.178989 77.3) (width 0.6) (layer "F.Cu") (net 6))
 (segment (start 131.178989 77.3) (end 131.5 77.3) (width 0.6) (layer "F.Cu") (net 6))
 (segment (start 124.966 75.206) (end 121.959032 75.206) (width 0.2) (layer "F.Cu") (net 7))
 (segment (start 122.975 72.065) (end 121.775 72.065) (width 0.2) (layer "F.Cu") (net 7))
 (segment (start 124.175 72.065) (end 124.375 71.865) (width 0.2) (layer "F.Cu") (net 7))
 (segment (start 121.475 74.721968) (end 121.475 74.4) (width 0.2) (layer "F.Cu") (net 7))
 (segment (start 121.775 72.065) (end 121.475 72.365) (width 0.2) (layer "F.Cu") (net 7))
 (segment (start 126.17 68.605) (end 126.175 68.6) (width 0.6) (layer "F.Cu") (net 7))
 (segment (start 122.975 72.065) (end 124.175 72.065) (width 0.2) (layer "F.Cu") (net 7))
 (segment (start 121.959032 75.206) (end 121.475 74.721968) (width 0.2) (layer "F.Cu") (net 7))
 (segment (start 121.475 72.365) (end 121.475 74.721968) (width 0.2) (layer "F.Cu") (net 7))
 (segment (start 124.375 71.865) (end 124.375 68.805) (width 0.2) (layer "F.Cu") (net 7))
 (segment (start 122.975 68.605) (end 126.17 68.605) (width 0.6) (layer "F.Cu") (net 7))
 (segment (start 126.96 77.2) (end 124.966 75.206) (width 0.2) (layer "F.Cu") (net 7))
 (segment (start 121.775 70.795) (end 121.075 71.495) (width 0.2) (layer "F.Cu") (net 8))
 (segment (start 124.975 67.335) (end 122.975 67.335) (width 0.6) (layer "F.Cu") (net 8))
 (segment (start 121.792932 75.607) (end 121.075 74.889068) (width 0.2) (layer "F.Cu") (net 8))
 (segment (start 121.075 68.035) (end 121.075 71.495) (width 0.2) (layer "F.Cu") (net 8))
 (segment (start 122.827 75.607) (end 121.792932 75.607) (width 0.2) (layer "F.Cu") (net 8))
 (segment (start 122.975 70.795) (end 121.775 70.795) (width 0.2) (layer "F.Cu") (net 8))
 (segment (start 122.975 67.335) (end 121.775 67.335) (width 0.2) (layer "F.Cu") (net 8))
 (segment (start 121.075 71.495) (end 121.075 74.889068) (width 0.2) (layer "F.Cu") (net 8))
 (segment (start 122.975 70.795) (end 122.000001 70.795) (width 0.2) (layer "F.Cu") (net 8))
 (segment (start 121.775 67.335) (end 121.075 68.035) (width 0.2) (layer "F.Cu") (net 8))
 (segment (start 124.42 77.2) (end 122.827 75.607) (width 0.2) (layer "F.Cu") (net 8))
 (segment (start 121.88 77.2) (end 119.975 75.295) (width 0.2) (layer "F.Cu") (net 4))
 (segment (start 119.975 75.295) (end 119.975 74.065) (width 0.2) (layer "F.Cu") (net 4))
 (segment (start 118.025 73.335) (end 116.125 73.335) (width 0.6) (layer "F.Cu") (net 4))
 (segment (start 119.975 74.065) (end 119.245 73.335) (width 0.2) (layer "F.Cu") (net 4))
 (segment (start 119.245 73.335) (end 118.025 73.335) (width 0.2) (layer "F.Cu") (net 4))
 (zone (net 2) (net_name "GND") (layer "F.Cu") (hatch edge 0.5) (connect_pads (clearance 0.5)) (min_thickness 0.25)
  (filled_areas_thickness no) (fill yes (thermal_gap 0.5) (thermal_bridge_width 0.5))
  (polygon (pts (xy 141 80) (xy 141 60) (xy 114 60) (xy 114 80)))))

